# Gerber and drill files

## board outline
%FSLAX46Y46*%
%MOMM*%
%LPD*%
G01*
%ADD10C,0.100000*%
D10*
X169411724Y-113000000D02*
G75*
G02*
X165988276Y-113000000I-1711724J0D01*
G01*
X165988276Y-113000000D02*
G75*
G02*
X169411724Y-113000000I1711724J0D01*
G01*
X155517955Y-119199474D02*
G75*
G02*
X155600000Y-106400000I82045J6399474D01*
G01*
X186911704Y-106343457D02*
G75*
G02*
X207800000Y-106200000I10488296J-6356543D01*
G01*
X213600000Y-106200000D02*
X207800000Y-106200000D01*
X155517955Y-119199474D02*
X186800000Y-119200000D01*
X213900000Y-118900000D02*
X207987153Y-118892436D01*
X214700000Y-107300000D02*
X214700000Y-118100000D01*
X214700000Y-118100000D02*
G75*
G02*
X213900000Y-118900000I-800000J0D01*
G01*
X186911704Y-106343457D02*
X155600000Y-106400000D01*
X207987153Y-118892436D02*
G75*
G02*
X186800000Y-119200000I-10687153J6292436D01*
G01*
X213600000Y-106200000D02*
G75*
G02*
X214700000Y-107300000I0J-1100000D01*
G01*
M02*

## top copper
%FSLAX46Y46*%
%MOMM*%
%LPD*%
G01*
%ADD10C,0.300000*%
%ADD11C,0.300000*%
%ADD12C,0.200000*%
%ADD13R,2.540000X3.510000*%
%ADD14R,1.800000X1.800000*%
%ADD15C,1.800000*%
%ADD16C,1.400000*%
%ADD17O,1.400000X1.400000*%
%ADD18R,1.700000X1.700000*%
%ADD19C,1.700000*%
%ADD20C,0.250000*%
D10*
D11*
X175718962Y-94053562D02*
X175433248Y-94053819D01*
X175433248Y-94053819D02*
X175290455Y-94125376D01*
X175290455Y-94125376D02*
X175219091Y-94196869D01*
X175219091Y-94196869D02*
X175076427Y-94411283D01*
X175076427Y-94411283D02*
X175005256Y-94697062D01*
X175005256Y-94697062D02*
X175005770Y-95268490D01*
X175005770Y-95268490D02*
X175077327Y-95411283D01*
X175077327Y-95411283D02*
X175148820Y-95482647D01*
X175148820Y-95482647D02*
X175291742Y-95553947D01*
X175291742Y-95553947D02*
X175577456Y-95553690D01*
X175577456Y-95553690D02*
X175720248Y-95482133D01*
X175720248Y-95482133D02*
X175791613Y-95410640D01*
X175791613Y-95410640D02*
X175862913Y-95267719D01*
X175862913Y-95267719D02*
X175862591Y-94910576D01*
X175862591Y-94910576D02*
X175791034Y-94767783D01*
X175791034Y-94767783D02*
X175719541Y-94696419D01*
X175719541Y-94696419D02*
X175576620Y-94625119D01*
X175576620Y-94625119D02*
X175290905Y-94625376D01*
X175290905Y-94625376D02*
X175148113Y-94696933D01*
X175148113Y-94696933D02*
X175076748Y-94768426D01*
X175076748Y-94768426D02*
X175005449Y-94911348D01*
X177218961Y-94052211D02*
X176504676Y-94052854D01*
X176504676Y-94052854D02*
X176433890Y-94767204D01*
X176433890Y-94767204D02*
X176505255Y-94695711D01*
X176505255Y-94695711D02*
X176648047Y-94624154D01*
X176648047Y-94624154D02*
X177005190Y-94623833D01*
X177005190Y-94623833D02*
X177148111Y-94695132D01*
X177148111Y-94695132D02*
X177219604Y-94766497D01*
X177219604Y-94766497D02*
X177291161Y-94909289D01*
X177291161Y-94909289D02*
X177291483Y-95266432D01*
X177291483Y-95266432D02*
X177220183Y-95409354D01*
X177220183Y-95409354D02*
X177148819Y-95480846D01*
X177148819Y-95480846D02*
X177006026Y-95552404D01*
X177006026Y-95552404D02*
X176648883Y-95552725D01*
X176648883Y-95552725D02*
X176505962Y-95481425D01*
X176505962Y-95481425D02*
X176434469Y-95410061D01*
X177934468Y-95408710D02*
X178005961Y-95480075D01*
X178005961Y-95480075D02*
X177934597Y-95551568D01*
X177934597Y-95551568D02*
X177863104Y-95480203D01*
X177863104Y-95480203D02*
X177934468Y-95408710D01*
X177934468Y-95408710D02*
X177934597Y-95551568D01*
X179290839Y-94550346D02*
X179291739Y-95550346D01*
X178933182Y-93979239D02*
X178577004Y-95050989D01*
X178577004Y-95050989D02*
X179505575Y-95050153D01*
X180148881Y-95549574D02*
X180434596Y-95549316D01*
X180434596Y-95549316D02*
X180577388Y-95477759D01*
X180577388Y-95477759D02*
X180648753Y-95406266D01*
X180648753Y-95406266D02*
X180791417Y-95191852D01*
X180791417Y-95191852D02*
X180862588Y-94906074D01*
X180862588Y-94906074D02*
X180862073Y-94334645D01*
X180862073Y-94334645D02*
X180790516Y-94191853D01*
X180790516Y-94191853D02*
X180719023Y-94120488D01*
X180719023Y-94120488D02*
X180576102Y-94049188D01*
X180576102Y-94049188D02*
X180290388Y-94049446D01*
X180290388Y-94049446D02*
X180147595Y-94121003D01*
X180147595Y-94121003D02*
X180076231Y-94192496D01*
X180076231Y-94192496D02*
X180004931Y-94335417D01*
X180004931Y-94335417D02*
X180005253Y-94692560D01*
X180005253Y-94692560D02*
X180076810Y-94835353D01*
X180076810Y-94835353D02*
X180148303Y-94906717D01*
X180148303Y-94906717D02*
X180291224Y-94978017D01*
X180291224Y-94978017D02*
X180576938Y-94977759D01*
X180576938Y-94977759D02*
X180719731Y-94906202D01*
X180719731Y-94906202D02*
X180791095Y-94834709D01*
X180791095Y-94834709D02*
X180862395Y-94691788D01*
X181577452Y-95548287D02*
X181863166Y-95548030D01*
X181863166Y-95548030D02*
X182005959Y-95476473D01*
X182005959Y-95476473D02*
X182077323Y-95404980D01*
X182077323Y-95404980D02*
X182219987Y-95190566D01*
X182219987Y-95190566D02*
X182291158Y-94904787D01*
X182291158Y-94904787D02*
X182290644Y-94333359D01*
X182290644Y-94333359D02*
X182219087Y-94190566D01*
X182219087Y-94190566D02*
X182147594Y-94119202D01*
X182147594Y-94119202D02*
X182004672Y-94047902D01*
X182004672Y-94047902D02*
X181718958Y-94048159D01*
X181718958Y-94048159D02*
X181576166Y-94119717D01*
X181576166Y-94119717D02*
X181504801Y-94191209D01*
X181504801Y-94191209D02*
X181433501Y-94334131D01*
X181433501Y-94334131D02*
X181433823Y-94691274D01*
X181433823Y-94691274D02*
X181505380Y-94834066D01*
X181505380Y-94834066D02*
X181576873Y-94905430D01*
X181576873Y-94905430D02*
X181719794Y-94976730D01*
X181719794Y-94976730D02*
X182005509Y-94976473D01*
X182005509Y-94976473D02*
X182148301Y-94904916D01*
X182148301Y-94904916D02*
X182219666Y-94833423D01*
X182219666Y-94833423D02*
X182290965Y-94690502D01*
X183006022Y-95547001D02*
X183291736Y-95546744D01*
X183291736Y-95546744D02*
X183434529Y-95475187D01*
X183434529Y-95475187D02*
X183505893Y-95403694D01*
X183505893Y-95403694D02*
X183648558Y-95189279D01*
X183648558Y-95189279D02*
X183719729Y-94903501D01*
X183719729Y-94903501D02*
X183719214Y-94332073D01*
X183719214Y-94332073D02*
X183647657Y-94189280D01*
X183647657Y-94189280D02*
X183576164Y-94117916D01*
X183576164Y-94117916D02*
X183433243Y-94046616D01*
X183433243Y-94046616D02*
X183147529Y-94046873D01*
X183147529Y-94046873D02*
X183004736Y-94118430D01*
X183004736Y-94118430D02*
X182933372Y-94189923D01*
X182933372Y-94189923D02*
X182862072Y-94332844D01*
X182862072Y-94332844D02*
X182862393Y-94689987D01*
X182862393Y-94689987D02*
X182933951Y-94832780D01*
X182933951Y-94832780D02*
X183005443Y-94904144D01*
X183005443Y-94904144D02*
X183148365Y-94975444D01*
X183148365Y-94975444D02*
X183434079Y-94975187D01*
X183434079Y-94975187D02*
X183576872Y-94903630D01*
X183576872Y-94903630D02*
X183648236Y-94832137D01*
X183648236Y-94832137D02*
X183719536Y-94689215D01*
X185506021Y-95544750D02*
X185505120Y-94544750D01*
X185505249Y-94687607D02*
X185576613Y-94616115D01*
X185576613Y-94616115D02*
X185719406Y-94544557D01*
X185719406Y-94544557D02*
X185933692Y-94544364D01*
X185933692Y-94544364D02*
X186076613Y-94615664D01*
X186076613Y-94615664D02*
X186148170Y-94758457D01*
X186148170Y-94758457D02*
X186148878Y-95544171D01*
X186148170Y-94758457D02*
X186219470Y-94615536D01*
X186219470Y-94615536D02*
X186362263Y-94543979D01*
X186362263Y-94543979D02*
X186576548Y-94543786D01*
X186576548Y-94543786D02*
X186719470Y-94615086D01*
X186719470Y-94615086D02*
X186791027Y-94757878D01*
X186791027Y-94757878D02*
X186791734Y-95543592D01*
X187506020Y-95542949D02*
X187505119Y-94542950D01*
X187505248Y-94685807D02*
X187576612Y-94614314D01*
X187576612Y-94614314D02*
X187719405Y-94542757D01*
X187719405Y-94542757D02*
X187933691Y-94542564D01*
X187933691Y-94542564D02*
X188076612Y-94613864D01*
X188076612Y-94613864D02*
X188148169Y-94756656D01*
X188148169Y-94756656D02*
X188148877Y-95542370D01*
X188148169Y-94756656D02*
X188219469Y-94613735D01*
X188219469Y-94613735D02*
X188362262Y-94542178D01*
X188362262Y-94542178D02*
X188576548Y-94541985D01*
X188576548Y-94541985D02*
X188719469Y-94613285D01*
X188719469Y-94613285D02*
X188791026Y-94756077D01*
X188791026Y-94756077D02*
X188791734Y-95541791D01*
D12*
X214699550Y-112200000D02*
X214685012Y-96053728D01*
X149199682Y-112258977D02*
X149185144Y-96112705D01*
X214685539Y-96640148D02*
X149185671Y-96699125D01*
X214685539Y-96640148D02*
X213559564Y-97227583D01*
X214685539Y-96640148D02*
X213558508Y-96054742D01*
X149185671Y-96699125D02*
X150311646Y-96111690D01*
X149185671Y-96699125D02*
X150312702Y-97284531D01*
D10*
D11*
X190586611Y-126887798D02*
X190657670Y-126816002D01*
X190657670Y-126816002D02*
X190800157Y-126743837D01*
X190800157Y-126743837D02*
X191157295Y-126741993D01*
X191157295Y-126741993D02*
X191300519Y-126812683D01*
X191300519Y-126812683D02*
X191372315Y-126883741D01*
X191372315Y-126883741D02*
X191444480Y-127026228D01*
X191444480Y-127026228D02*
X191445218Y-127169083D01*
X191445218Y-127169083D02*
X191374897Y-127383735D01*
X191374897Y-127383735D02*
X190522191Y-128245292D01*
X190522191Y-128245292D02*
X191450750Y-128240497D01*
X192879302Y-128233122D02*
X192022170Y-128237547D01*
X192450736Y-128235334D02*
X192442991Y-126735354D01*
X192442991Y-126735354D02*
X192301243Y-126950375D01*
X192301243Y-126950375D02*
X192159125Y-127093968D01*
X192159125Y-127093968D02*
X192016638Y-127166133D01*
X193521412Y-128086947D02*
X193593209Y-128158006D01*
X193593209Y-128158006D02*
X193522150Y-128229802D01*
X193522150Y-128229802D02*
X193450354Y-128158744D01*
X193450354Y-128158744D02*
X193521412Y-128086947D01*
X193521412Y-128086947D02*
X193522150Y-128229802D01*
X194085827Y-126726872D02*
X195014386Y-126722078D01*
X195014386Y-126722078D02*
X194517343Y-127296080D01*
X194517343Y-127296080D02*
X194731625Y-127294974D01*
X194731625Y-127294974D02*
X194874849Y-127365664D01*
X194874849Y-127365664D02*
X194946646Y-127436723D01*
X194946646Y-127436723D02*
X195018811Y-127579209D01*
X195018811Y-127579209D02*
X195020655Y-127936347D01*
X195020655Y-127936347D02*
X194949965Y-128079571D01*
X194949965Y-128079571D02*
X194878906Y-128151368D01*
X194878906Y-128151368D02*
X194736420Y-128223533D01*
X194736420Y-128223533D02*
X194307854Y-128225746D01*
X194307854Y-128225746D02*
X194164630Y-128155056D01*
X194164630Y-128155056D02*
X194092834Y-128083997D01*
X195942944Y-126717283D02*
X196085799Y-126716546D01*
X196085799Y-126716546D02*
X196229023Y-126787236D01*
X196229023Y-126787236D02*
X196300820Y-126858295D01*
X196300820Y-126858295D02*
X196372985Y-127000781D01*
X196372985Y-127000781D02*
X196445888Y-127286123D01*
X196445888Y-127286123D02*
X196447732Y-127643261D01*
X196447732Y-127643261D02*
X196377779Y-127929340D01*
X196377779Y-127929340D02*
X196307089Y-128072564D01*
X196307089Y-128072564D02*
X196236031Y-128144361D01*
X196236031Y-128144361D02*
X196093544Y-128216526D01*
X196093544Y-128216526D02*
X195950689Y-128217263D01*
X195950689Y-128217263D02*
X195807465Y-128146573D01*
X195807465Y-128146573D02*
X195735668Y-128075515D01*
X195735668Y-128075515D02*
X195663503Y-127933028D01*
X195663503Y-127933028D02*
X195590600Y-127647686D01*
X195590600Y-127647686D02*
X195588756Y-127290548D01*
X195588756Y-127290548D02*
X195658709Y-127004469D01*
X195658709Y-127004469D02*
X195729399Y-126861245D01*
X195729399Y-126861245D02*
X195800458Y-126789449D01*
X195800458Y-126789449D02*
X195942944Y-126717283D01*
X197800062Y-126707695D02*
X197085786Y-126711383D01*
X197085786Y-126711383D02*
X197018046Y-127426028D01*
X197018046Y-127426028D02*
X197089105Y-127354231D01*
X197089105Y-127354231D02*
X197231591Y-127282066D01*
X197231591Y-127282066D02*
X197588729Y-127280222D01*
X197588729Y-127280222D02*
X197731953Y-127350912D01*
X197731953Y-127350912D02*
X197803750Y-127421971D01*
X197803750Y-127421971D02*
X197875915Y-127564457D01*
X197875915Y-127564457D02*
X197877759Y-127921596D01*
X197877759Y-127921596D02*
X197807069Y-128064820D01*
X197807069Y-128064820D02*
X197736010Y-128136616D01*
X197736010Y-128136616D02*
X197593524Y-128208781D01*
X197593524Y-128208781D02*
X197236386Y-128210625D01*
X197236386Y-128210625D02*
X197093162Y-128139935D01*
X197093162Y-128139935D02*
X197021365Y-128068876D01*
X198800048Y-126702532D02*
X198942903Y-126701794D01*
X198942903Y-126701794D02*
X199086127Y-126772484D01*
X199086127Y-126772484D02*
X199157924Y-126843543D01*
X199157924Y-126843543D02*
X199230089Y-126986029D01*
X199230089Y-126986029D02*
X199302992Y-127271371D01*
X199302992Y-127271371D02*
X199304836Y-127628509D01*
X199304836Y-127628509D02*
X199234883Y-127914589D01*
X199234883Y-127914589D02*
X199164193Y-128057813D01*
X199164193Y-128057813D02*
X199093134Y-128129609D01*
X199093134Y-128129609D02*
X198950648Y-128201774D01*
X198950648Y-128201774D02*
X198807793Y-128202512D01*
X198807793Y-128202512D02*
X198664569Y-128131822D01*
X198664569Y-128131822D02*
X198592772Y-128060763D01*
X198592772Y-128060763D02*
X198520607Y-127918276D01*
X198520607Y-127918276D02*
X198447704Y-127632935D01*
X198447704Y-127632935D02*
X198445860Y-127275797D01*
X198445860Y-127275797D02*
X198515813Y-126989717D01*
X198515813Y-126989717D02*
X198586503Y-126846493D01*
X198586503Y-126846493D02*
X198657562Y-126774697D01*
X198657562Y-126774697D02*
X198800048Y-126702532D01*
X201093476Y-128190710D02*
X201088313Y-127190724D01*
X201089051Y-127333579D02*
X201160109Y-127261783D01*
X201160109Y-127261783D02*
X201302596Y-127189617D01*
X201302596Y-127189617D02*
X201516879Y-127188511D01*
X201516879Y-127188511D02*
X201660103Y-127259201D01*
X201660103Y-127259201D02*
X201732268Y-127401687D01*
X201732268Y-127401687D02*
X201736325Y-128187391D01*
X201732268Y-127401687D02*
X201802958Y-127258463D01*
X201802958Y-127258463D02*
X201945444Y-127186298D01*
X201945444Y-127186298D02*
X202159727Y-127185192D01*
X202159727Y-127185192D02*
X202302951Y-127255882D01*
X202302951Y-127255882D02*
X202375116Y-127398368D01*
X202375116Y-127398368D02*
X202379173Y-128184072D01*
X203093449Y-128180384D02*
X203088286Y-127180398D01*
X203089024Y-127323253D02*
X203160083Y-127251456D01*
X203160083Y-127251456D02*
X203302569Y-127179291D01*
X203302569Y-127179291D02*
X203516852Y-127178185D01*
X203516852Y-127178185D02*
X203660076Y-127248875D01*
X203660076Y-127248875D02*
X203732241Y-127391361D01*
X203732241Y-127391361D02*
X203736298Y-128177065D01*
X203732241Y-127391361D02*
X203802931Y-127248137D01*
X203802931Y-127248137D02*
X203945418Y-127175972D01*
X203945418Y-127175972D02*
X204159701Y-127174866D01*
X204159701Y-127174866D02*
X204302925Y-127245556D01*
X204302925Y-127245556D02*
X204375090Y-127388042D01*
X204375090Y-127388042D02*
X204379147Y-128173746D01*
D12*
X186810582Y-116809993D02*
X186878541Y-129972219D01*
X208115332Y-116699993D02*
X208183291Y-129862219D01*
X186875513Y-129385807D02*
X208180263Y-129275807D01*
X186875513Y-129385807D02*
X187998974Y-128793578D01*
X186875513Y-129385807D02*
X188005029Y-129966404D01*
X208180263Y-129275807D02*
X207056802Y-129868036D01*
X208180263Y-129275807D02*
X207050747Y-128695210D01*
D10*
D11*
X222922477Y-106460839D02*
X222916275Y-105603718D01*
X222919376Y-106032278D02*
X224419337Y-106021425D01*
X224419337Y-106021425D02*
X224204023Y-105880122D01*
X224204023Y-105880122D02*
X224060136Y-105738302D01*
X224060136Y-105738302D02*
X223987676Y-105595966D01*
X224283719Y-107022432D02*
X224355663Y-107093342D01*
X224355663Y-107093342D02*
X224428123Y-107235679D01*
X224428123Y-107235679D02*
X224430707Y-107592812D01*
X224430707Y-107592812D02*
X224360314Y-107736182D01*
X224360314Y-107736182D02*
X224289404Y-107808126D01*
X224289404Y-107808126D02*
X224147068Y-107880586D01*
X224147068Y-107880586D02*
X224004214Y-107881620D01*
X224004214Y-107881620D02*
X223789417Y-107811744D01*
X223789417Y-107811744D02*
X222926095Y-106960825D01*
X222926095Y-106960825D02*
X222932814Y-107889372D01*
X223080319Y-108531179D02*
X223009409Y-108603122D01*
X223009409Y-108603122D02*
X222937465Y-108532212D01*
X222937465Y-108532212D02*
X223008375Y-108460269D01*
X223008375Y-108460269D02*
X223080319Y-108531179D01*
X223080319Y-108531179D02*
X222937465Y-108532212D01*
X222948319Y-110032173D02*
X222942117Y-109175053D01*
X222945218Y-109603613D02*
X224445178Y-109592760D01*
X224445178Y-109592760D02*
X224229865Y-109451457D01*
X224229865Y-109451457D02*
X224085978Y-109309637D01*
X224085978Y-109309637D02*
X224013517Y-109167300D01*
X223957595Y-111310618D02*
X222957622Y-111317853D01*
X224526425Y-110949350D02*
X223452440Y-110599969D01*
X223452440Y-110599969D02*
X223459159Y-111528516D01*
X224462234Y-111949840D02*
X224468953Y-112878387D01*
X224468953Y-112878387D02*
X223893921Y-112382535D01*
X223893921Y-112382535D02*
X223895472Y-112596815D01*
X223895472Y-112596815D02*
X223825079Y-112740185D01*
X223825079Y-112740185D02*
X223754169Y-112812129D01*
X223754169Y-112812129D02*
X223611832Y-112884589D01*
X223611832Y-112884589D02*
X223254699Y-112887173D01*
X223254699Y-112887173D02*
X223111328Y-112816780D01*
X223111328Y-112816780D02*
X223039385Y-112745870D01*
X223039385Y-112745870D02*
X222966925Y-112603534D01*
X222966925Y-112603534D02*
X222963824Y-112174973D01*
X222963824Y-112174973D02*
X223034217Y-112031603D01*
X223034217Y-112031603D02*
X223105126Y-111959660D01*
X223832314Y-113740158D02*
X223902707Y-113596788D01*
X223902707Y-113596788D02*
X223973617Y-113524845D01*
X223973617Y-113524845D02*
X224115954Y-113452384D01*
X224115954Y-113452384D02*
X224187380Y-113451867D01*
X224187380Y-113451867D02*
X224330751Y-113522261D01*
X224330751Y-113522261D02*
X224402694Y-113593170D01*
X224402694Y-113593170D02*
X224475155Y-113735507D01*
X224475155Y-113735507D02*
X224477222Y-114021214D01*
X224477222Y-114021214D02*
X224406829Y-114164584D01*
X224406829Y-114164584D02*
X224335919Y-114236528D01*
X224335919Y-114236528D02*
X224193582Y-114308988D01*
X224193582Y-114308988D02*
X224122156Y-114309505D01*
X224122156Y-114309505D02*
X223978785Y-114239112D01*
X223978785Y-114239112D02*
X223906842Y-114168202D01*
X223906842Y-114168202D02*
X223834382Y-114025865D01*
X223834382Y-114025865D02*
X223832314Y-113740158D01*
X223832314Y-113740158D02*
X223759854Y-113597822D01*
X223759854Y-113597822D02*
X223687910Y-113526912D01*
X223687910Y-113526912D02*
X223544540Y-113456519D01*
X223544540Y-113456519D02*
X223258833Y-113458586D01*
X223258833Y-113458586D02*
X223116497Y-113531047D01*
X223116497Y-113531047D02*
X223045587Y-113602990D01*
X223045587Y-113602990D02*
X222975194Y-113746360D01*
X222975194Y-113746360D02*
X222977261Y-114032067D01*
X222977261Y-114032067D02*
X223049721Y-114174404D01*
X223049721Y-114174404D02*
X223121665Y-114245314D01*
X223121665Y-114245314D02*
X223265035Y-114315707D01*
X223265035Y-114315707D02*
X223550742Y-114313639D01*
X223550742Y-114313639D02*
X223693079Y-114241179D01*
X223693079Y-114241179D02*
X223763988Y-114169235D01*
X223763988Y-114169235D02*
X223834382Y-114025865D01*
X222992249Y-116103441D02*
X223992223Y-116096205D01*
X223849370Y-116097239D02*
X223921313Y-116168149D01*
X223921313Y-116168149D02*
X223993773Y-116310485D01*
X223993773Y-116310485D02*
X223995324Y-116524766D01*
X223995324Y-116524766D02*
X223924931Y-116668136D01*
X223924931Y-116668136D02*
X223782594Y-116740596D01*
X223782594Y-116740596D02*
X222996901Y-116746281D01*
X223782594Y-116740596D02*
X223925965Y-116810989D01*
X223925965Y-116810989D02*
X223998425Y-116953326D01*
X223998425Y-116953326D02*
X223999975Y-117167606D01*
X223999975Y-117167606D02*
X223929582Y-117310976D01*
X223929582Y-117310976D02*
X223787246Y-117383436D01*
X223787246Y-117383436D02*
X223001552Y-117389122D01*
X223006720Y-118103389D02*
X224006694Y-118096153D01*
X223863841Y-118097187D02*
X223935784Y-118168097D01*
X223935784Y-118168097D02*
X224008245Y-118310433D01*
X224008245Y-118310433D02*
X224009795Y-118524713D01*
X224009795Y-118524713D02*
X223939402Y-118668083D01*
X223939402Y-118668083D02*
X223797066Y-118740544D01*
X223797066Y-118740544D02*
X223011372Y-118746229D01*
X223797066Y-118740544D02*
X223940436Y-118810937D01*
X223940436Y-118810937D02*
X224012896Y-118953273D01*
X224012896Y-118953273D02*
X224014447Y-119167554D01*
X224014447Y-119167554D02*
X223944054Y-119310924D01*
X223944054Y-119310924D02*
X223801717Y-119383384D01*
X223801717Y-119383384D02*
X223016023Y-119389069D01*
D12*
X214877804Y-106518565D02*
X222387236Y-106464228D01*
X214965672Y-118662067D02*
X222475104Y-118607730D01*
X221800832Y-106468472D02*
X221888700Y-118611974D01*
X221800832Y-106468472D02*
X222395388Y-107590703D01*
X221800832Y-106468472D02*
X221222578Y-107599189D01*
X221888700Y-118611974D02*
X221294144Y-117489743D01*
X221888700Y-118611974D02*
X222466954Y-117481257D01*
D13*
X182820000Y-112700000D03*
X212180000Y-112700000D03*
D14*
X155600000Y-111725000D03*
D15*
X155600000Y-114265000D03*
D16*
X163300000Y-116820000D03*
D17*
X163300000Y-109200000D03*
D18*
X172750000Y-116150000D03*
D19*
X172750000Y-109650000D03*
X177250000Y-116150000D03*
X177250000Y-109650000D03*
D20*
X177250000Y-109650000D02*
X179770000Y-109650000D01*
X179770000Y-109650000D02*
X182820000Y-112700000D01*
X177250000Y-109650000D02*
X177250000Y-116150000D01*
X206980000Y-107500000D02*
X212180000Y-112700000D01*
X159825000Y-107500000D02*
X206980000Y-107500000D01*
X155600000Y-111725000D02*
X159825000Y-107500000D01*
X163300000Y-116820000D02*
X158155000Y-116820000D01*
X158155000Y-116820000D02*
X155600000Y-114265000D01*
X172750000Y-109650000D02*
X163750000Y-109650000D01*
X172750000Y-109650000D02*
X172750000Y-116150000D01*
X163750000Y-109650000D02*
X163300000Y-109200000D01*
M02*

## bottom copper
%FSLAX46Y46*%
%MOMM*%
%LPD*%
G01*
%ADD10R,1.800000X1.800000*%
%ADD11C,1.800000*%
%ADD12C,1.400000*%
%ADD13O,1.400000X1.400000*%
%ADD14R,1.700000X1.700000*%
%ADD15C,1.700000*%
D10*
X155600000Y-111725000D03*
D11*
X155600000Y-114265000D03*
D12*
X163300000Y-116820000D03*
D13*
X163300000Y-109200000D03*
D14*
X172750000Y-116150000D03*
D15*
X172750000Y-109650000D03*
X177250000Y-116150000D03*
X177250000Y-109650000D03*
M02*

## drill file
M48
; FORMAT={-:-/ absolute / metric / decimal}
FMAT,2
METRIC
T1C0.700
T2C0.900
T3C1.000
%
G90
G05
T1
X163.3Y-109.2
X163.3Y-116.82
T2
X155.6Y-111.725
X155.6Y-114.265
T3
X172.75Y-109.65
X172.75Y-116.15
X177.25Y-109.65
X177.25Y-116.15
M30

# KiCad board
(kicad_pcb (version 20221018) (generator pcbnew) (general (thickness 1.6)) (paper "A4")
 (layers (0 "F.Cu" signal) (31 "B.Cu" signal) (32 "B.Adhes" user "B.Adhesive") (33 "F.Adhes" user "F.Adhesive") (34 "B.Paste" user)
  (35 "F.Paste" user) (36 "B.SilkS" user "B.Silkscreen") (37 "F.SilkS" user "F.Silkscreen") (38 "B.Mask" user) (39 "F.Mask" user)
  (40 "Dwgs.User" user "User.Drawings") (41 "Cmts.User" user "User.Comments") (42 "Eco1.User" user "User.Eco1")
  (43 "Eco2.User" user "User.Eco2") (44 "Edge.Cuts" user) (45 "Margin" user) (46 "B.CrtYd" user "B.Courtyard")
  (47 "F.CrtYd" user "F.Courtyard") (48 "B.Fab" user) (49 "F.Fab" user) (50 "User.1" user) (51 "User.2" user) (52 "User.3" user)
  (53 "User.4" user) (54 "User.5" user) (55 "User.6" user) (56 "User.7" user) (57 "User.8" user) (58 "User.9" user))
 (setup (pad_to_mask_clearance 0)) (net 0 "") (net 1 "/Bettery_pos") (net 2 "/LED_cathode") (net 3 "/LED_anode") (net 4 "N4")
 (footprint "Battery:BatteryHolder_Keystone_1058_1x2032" (layer "F.Cu") (at 197.5 112.7)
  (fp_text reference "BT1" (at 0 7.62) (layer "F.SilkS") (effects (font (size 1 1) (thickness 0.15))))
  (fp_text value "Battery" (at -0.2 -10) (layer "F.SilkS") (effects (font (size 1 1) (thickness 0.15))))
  (pad "1" smd rect (at -14.68 0) (size 2.54 3.51) (layers "F.Cu" "F.Paste" "F.Mask") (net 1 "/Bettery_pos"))
  (pad "2" smd rect (at 14.68 0) (size 2.54 3.51) (layers "F.Cu" "F.Paste" "F.Mask") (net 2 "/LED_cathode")))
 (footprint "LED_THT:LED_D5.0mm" (layer "F.Cu") (at 155.6 111.725 -90)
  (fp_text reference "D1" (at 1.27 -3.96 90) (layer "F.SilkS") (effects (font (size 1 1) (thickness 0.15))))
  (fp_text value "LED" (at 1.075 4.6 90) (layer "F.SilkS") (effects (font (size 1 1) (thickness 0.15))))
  (pad "1" thru_hole rect (at 0 0 270) (size 1.8 1.8) (drill 0.9) (layers "*.Cu" "*.Mask") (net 2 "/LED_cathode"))
  (pad "2" thru_hole circle (at 2.54 0 270) (size 1.8 1.8) (drill 0.9) (layers "*.Cu" "*.Mask") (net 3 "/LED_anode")))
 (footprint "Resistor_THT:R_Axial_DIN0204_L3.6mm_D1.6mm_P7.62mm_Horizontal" (layer "F.Cu") (at 163.3 116.82 90)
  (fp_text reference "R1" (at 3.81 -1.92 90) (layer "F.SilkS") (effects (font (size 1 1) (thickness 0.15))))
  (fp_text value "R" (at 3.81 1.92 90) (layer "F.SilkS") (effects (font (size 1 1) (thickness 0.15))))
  (pad "1" thru_hole circle (at 0 0 90) (size 1.4 1.4) (drill 0.7) (layers "*.Cu" "*.Mask") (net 3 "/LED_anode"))
  (pad "2" thru_hole oval (at 7.62 0 90) (size 1.4 1.4) (drill 0.7) (layers "*.Cu" "*.Mask") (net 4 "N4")))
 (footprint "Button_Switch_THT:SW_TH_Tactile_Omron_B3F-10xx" (layer "F.Cu") (at 172.75 116.15 90)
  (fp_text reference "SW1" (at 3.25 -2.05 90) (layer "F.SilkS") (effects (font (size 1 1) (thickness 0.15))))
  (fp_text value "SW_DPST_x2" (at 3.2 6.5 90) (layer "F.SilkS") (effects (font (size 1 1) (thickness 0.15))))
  (pad "1" thru_hole rect (at 0 0 90) (size 1.7 1.7) (drill 1) (layers "*.Cu" "*.Mask") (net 4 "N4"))
  (pad "1" thru_hole circle (at 6.5 0 90) (size 1.7 1.7) (drill 1) (layers "*.Cu" "*.Mask") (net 4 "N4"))
  (pad "2" thru_hole circle (at 0 4.5 90) (size 1.7 1.7) (drill 1) (layers "*.Cu" "*.Mask") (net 1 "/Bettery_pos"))
  (pad "2" thru_hole circle (at 6.5 4.5 90) (size 1.7 1.7) (drill 1) (layers "*.Cu" "*.Mask") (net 1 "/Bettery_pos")))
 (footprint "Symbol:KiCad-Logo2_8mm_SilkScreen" (layer "B.Cu") (at 197.8 111.9 180)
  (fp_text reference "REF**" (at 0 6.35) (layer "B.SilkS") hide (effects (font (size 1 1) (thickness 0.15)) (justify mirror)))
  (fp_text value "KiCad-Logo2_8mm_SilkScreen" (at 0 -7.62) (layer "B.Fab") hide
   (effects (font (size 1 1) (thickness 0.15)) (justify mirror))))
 (gr_circle (center 167.7 113) (end 166 112.8) (stroke (width 0.1) (type default)) (fill none) (layer "Edge.Cuts"))
 (gr_arc (start 155.517955 119.199474) (mid 149.200132 112.758977) (end 155.6 106.4) (stroke (width 0.1) (type default)) (layer "Edge.Cuts"))
 (gr_arc (start 186.911704 106.343457) (mid 197.315774 100.436114) (end 207.8 106.2) (stroke (width 0.1) (type default)) (layer "Edge.Cuts"))
 (gr_line (start 213.6 106.2) (end 207.8 106.2) (stroke (width 0.1) (type default)) (layer "Edge.Cuts"))
 (gr_line (start 155.517955 119.199474) (end 186.8 119.2) (stroke (width 0.1) (type default)) (layer "Edge.Cuts"))
 (gr_line (start 213.9 118.9) (end 207.987153 118.892436) (stroke (width 0.1) (type default)) (layer "Edge.Cuts"))
 (gr_line (start 214.7 107.3) (end 214.7 118.1) (stroke (width 0.1) (type default)) (layer "Edge.Cuts"))
 (gr_arc (start 214.7 118.1) (mid 214.465685 118.665685) (end 213.9 118.9) (stroke (width 0.1) (type default)) (layer "Edge.Cuts"))
 (gr_line (start 186.911704 106.343457) (end 155.6 106.4) (stroke (width 0.1) (type default)) (layer "Edge.Cuts"))
 (gr_arc (start 207.987153 118.892436) (mid 197.480015 125.000709) (end 186.800001 119.199999) (stroke (width 0.1) (type default))
  (layer "Edge.Cuts"))
 (gr_arc (start 213.6 106.2) (mid 214.377817 106.522183) (end 214.7 107.3) (stroke (width 0.1) (type default)) (layer "Edge.Cuts"))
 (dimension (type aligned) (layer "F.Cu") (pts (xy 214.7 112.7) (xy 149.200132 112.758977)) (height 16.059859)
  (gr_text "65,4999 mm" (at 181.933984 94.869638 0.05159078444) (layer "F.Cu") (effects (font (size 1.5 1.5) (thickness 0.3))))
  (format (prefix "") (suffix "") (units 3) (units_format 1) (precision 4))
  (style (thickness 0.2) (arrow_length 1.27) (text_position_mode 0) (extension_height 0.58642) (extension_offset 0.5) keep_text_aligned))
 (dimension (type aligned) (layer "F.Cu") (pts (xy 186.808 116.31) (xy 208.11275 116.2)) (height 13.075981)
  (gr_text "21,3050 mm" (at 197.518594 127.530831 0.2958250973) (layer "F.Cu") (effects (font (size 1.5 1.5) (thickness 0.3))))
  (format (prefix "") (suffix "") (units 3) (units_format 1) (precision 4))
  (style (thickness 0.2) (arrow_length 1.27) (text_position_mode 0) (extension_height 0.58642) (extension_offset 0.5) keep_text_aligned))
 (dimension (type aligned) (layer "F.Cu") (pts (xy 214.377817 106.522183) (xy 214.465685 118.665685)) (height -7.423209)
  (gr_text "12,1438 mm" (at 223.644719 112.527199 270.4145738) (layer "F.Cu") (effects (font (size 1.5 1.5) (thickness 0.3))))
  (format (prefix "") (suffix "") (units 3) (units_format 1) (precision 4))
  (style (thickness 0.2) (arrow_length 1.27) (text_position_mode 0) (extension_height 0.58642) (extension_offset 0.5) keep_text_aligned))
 (segment (start 177.25 109.65) (end 179.77 109.65) (width 0.25) (layer "F.Cu") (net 1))
 (segment (start 179.77 109.65) (end 182.82 112.7) (width 0.25) (layer "F.Cu") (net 1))
 (segment (start 177.25 109.65) (end 177.25 116.15) (width 0.25) (layer "F.Cu") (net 1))
 (segment (start 206.98 107.5) (end 212.18 112.7) (width 0.25) (layer "F.Cu") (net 2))
 (segment (start 159.825 107.5) (end 206.98 107.5) (width 0.25) (layer "F.Cu") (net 2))
 (segment (start 155.6 111.725) (end 159.825 107.5) (width 0.25) (layer "F.Cu") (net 2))
 (segment (start 163.3 116.82) (end 158.155 116.82) (width 0.25) (layer "F.Cu") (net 3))
 (segment (start 158.155 116.82) (end 155.6 114.265) (width 0.25) (layer "F.Cu") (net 3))
 (segment (start 172.75 109.65) (end 163.75 109.65) (width 0.25) (layer "F.Cu") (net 4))
 (segment (start 172.75 109.65) (end 172.75 116.15) (width 0.25) (layer "F.Cu") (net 4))
 (segment (start 163.75 109.65) (end 163.3 109.2) (width 0.25) (layer "F.Cu") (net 4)))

